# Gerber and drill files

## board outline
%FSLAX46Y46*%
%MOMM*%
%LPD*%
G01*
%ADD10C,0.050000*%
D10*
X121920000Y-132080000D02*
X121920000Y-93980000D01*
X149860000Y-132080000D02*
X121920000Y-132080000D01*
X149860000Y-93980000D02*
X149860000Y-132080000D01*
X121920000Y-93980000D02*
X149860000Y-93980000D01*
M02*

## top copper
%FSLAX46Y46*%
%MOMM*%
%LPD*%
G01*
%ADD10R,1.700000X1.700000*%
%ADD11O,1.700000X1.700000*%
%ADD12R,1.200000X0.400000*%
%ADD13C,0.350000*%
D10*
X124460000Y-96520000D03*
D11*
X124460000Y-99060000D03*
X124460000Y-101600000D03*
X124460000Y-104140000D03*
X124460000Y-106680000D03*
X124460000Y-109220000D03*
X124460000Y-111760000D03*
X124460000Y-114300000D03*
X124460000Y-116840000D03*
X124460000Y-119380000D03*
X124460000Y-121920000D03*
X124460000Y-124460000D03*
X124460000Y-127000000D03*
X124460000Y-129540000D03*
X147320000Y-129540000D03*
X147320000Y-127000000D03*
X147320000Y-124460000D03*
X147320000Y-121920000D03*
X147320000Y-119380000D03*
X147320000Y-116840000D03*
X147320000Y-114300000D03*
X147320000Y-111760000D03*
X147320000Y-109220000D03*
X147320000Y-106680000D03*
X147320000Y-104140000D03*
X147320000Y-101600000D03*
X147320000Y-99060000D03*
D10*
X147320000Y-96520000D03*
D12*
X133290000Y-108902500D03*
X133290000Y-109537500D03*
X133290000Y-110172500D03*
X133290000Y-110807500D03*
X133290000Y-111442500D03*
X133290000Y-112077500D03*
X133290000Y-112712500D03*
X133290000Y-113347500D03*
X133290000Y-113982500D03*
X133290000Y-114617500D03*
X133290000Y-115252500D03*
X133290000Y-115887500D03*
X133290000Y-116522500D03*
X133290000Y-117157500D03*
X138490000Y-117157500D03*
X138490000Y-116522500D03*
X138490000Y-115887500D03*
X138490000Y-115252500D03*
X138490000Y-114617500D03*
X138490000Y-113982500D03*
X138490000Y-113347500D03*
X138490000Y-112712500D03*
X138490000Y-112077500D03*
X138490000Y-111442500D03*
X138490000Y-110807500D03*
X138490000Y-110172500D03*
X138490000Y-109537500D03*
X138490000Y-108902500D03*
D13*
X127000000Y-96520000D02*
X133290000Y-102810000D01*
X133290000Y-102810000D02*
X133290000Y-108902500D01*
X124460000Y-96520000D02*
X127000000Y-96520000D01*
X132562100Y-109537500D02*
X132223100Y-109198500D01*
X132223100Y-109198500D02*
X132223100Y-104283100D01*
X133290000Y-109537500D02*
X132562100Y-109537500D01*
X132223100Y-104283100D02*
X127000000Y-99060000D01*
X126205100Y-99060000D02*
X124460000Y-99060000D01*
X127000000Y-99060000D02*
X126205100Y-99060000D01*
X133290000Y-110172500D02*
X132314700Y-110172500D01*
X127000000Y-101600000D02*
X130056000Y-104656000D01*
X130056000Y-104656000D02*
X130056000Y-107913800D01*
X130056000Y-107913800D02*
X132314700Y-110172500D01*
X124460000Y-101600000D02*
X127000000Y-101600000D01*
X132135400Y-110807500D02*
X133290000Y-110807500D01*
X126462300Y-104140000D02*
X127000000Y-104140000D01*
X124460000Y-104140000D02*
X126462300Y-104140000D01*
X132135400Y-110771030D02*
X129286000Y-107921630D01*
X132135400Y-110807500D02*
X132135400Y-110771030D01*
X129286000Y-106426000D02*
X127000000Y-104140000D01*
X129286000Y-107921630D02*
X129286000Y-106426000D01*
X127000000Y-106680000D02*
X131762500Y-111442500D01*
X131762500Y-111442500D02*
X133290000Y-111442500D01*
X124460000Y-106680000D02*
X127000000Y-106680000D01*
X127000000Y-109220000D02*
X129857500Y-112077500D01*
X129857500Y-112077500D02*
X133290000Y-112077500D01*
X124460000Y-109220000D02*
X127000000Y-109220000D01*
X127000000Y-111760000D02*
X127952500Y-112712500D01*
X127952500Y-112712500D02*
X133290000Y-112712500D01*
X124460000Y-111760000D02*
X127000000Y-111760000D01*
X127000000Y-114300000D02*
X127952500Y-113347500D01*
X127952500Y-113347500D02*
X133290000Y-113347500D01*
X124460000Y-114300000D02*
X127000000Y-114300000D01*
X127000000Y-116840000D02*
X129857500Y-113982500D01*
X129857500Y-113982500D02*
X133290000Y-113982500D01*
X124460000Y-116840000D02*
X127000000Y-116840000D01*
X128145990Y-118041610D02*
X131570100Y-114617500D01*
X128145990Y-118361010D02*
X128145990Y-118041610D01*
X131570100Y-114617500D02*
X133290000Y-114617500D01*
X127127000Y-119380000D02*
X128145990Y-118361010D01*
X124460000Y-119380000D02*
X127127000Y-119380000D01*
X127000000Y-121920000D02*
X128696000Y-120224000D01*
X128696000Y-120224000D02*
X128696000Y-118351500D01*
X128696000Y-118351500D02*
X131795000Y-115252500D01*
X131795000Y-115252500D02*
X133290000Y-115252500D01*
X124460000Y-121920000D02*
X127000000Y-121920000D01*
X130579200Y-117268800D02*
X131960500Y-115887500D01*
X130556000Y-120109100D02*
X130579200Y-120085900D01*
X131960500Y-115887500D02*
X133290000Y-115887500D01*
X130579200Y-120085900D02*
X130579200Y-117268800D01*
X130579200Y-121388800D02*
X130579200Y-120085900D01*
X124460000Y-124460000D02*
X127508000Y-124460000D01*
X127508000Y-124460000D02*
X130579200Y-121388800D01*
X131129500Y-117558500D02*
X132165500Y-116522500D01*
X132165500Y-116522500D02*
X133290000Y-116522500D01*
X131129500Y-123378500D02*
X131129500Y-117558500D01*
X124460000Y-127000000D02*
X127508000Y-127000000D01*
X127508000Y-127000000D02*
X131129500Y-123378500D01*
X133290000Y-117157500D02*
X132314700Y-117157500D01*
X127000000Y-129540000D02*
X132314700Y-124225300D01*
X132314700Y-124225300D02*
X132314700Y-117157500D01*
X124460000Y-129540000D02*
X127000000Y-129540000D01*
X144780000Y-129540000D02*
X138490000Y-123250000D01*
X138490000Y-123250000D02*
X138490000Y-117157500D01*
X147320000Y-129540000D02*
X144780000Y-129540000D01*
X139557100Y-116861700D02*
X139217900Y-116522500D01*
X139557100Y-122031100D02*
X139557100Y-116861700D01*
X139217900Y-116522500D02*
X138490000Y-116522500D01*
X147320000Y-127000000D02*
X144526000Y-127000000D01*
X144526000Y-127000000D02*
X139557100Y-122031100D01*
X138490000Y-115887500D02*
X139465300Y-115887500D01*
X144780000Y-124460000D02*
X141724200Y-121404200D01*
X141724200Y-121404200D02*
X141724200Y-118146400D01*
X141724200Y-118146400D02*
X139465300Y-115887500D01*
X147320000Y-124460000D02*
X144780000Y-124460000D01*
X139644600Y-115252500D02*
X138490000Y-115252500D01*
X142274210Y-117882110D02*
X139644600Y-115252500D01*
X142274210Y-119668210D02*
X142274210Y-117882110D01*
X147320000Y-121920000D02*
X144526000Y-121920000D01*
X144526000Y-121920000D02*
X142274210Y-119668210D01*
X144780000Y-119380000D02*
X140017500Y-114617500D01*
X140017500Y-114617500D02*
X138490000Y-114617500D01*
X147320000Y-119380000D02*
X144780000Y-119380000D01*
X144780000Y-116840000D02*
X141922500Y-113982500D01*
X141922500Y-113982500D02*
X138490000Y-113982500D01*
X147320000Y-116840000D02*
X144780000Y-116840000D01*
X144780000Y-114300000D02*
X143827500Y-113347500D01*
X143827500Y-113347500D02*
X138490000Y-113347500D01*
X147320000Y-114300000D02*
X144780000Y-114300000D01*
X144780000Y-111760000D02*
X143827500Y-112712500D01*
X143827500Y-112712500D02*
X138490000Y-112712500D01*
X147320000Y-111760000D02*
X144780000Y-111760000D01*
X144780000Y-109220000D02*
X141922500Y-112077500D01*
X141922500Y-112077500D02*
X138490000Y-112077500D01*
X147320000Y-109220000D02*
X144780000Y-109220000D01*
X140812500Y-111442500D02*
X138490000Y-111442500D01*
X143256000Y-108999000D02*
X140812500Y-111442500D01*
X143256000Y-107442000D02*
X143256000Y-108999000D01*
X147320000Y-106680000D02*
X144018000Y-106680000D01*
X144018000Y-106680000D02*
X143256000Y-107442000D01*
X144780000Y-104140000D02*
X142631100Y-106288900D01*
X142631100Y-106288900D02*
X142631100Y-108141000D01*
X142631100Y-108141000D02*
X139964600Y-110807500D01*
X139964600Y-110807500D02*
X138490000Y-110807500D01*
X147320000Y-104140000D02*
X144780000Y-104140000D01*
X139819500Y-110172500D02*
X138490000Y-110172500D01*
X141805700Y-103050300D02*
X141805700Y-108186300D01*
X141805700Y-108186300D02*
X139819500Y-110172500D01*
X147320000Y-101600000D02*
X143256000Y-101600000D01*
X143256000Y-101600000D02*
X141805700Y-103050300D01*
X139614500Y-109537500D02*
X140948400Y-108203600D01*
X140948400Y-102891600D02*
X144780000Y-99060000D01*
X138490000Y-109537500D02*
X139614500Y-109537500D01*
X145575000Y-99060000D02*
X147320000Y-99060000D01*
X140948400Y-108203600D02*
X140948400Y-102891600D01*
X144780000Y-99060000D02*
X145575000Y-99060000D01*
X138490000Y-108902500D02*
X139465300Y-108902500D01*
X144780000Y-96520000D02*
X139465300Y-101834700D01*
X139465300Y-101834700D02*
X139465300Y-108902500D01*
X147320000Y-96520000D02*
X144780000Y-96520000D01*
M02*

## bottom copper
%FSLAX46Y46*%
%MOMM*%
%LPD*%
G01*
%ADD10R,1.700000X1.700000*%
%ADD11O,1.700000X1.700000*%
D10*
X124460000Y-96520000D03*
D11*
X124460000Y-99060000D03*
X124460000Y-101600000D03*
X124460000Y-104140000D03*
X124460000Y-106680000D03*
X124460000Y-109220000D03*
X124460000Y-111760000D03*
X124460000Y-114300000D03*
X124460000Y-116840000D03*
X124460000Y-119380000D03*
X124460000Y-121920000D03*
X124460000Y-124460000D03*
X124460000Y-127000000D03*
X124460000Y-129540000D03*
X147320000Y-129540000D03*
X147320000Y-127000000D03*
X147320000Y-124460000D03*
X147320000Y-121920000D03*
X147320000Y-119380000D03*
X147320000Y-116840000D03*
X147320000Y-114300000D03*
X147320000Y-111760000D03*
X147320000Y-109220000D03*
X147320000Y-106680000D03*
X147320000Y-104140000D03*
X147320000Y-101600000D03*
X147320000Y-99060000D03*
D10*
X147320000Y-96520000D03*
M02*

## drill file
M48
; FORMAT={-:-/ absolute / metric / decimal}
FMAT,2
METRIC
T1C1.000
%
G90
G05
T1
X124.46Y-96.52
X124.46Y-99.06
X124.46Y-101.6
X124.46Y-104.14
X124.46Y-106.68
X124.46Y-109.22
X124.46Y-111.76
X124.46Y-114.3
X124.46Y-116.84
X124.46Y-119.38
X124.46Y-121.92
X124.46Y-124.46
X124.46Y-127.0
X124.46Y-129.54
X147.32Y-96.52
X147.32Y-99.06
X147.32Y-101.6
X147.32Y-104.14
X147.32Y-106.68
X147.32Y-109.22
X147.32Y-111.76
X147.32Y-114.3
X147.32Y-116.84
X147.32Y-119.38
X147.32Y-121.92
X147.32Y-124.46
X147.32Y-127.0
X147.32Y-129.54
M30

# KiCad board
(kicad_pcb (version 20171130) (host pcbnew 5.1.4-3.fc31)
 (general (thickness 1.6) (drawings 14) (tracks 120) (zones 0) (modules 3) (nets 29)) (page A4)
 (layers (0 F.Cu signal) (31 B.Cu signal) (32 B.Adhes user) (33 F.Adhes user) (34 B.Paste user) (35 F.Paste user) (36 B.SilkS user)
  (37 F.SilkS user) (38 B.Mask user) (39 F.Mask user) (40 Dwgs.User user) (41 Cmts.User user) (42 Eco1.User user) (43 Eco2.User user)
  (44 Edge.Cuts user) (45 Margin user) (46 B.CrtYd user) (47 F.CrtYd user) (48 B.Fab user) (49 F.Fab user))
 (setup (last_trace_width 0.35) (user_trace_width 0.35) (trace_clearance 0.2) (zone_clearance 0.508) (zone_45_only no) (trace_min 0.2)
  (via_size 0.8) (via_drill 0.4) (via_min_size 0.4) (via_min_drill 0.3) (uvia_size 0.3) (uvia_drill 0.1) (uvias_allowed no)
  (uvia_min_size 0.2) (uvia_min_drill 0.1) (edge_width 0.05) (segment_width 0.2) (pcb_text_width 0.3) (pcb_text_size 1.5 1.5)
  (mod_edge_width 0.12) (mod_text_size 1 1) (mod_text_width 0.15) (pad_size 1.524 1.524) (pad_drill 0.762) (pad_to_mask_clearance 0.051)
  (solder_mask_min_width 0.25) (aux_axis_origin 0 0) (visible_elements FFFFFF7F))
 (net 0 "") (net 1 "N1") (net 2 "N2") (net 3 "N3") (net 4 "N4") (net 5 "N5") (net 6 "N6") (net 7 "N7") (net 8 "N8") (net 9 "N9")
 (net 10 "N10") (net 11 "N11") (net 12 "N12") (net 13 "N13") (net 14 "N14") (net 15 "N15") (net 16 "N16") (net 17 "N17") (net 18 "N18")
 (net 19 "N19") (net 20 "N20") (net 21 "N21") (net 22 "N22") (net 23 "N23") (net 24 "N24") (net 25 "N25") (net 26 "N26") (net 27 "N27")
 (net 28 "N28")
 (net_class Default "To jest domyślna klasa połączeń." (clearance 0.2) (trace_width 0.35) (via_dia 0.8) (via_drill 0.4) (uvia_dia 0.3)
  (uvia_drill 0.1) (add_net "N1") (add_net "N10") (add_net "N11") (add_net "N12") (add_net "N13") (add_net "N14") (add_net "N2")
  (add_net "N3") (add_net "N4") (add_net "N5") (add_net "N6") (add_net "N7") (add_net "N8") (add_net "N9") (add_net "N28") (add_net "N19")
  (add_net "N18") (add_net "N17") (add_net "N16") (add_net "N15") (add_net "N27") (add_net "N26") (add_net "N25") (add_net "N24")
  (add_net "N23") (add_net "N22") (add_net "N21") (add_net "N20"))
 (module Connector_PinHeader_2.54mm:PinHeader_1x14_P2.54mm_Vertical (layer B.Cu) (at 124.46 96.52 180)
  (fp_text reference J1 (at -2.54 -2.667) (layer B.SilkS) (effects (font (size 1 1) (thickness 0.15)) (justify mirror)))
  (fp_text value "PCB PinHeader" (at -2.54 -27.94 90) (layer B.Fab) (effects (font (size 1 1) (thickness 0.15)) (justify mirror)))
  (pad 1 thru_hole rect (at 0 0 180) (size 1.7 1.7) (drill 1) (layers *.Cu *.Mask) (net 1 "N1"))
  (pad 2 thru_hole oval (at 0 -2.54 180) (size 1.7 1.7) (drill 1) (layers *.Cu *.Mask) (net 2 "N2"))
  (pad 3 thru_hole oval (at 0 -5.08 180) (size 1.7 1.7) (drill 1) (layers *.Cu *.Mask) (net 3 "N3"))
  (pad 4 thru_hole oval (at 0 -7.62 180) (size 1.7 1.7) (drill 1) (layers *.Cu *.Mask) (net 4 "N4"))
  (pad 5 thru_hole oval (at 0 -10.16 180) (size 1.7 1.7) (drill 1) (layers *.Cu *.Mask) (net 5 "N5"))
  (pad 6 thru_hole oval (at 0 -12.7 180) (size 1.7 1.7) (drill 1) (layers *.Cu *.Mask) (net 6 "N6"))
  (pad 7 thru_hole oval (at 0 -15.24 180) (size 1.7 1.7) (drill 1) (layers *.Cu *.Mask) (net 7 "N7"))
  (pad 8 thru_hole oval (at 0 -17.78 180) (size 1.7 1.7) (drill 1) (layers *.Cu *.Mask) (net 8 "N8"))
  (pad 9 thru_hole oval (at 0 -20.32 180) (size 1.7 1.7) (drill 1) (layers *.Cu *.Mask) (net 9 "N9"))
  (pad 10 thru_hole oval (at 0 -22.86 180) (size 1.7 1.7) (drill 1) (layers *.Cu *.Mask) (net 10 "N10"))
  (pad 11 thru_hole oval (at 0 -25.4 180) (size 1.7 1.7) (drill 1) (layers *.Cu *.Mask) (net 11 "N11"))
  (pad 12 thru_hole oval (at 0 -27.94 180) (size 1.7 1.7) (drill 1) (layers *.Cu *.Mask) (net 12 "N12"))
  (pad 13 thru_hole oval (at 0 -30.48 180) (size 1.7 1.7) (drill 1) (layers *.Cu *.Mask) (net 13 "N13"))
  (pad 14 thru_hole oval (at 0 -33.02 180) (size 1.7 1.7) (drill 1) (layers *.Cu *.Mask) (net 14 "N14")))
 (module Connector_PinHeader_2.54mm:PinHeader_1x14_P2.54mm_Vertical (layer B.Cu) (at 147.32 96.52 180)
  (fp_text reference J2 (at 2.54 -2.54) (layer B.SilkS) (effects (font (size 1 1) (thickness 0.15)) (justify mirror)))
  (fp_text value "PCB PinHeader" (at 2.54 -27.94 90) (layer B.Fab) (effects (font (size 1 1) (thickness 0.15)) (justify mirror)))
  (pad 14 thru_hole oval (at 0 -33.02 180) (size 1.7 1.7) (drill 1) (layers *.Cu *.Mask) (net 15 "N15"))
  (pad 13 thru_hole oval (at 0 -30.48 180) (size 1.7 1.7) (drill 1) (layers *.Cu *.Mask) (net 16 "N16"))
  (pad 12 thru_hole oval (at 0 -27.94 180) (size 1.7 1.7) (drill 1) (layers *.Cu *.Mask) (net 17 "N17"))
  (pad 11 thru_hole oval (at 0 -25.4 180) (size 1.7 1.7) (drill 1) (layers *.Cu *.Mask) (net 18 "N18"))
  (pad 10 thru_hole oval (at 0 -22.86 180) (size 1.7 1.7) (drill 1) (layers *.Cu *.Mask) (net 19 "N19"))
  (pad 9 thru_hole oval (at 0 -20.32 180) (size 1.7 1.7) (drill 1) (layers *.Cu *.Mask) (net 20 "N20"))
  (pad 8 thru_hole oval (at 0 -17.78 180) (size 1.7 1.7) (drill 1) (layers *.Cu *.Mask) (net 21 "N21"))
  (pad 7 thru_hole oval (at 0 -15.24 180) (size 1.7 1.7) (drill 1) (layers *.Cu *.Mask) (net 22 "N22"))
  (pad 6 thru_hole oval (at 0 -12.7 180) (size 1.7 1.7) (drill 1) (layers *.Cu *.Mask) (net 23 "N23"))
  (pad 5 thru_hole oval (at 0 -10.16 180) (size 1.7 1.7) (drill 1) (layers *.Cu *.Mask) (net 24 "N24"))
  (pad 4 thru_hole oval (at 0 -7.62 180) (size 1.7 1.7) (drill 1) (layers *.Cu *.Mask) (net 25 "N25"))
  (pad 3 thru_hole oval (at 0 -5.08 180) (size 1.7 1.7) (drill 1) (layers *.Cu *.Mask) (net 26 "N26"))
  (pad 2 thru_hole oval (at 0 -2.54 180) (size 1.7 1.7) (drill 1) (layers *.Cu *.Mask) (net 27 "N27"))
  (pad 1 thru_hole rect (at 0 0 180) (size 1.7 1.7) (drill 1) (layers *.Cu *.Mask) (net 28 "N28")))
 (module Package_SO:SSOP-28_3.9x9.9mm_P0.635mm (layer F.Cu) (at 135.89 113.03)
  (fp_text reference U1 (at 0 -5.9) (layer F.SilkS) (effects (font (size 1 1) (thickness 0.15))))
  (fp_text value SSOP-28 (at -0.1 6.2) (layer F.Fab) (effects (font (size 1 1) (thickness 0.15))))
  (pad 1 smd rect (at -2.6 -4.1275) (size 1.2 0.4) (layers F.Cu F.Paste F.Mask) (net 1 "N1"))
  (pad 2 smd rect (at -2.6 -3.4925) (size 1.2 0.4) (layers F.Cu F.Paste F.Mask) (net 2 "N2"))
  (pad 3 smd rect (at -2.6 -2.8575) (size 1.2 0.4) (layers F.Cu F.Paste F.Mask) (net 3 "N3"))
  (pad 4 smd rect (at -2.6 -2.2225) (size 1.2 0.4) (layers F.Cu F.Paste F.Mask) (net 4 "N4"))
  (pad 5 smd rect (at -2.6 -1.5875) (size 1.2 0.4) (layers F.Cu F.Paste F.Mask) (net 5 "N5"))
  (pad 6 smd rect (at -2.6 -0.9525) (size 1.2 0.4) (layers F.Cu F.Paste F.Mask) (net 6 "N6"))
  (pad 7 smd rect (at -2.6 -0.3175) (size 1.2 0.4) (layers F.Cu F.Paste F.Mask) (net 7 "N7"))
  (pad 8 smd rect (at -2.6 0.3175) (size 1.2 0.4) (layers F.Cu F.Paste F.Mask) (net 8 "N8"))
  (pad 9 smd rect (at -2.6 0.9525) (size 1.2 0.4) (layers F.Cu F.Paste F.Mask) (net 9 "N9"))
  (pad 10 smd rect (at -2.6 1.5875) (size 1.2 0.4) (layers F.Cu F.Paste F.Mask) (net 10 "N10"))
  (pad 11 smd rect (at -2.6 2.2225) (size 1.2 0.4) (layers F.Cu F.Paste F.Mask) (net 11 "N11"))
  (pad 12 smd rect (at -2.6 2.8575) (size 1.2 0.4) (layers F.Cu F.Paste F.Mask) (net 12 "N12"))
  (pad 13 smd rect (at -2.6 3.4925) (size 1.2 0.4) (layers F.Cu F.Paste F.Mask) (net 13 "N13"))
  (pad 14 smd rect (at -2.6 4.1275) (size 1.2 0.4) (layers F.Cu F.Paste F.Mask) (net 14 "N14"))
  (pad 15 smd rect (at 2.6 4.1275) (size 1.2 0.4) (layers F.Cu F.Paste F.Mask) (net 15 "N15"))
  (pad 16 smd rect (at 2.6 3.4925) (size 1.2 0.4) (layers F.Cu F.Paste F.Mask) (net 16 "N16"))
  (pad 17 smd rect (at 2.6 2.8575) (size 1.2 0.4) (layers F.Cu F.Paste F.Mask) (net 17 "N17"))
  (pad 18 smd rect (at 2.6 2.2225) (size 1.2 0.4) (layers F.Cu F.Paste F.Mask) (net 18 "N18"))
  (pad 19 smd rect (at 2.6 1.5875) (size 1.2 0.4) (layers F.Cu F.Paste F.Mask) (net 19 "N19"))
  (pad 20 smd rect (at 2.6 0.9525) (size 1.2 0.4) (layers F.Cu F.Paste F.Mask) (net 20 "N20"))
  (pad 21 smd rect (at 2.6 0.3175) (size 1.2 0.4) (layers F.Cu F.Paste F.Mask) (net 21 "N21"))
  (pad 22 smd rect (at 2.6 -0.3175) (size 1.2 0.4) (layers F.Cu F.Paste F.Mask) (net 22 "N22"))
  (pad 23 smd rect (at 2.6 -0.9525) (size 1.2 0.4) (layers F.Cu F.Paste F.Mask) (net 23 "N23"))
  (pad 24 smd rect (at 2.6 -1.5875) (size 1.2 0.4) (layers F.Cu F.Paste F.Mask) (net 24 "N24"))
  (pad 25 smd rect (at 2.6 -2.2225) (size 1.2 0.4) (layers F.Cu F.Paste F.Mask) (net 25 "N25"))
  (pad 26 smd rect (at 2.6 -2.8575) (size 1.2 0.4) (layers F.Cu F.Paste F.Mask) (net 26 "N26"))
  (pad 27 smd rect (at 2.6 -3.4925) (size 1.2 0.4) (layers F.Cu F.Paste F.Mask) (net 27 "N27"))
  (pad 28 smd rect (at 2.6 -4.1275) (size 1.2 0.4) (layers F.Cu F.Paste F.Mask) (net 28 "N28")))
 (gr_line (start 121.92 132.08) (end 121.92 93.98) (layer Edge.Cuts) (width 0.05))
 (gr_line (start 149.86 132.08) (end 121.92 132.08) (layer Edge.Cuts) (width 0.05))
 (gr_line (start 149.86 93.98) (end 149.86 132.08) (layer Edge.Cuts) (width 0.05))
 (gr_line (start 121.92 93.98) (end 149.86 93.98) (layer Edge.Cuts) (width 0.05))
 (segment (start 127 96.52) (end 133.29 102.81) (width 0.35) (layer F.Cu) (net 1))
 (segment (start 133.29 102.81) (end 133.29 108.9025) (width 0.35) (layer F.Cu) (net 1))
 (segment (start 124.46 96.52) (end 127 96.52) (width 0.35) (layer F.Cu) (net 1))
 (segment (start 132.5621 109.5375) (end 132.2231 109.1985) (width 0.35) (layer F.Cu) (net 2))
 (segment (start 132.2231 109.1985) (end 132.2231 104.2831) (width 0.35) (layer F.Cu) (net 2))
 (segment (start 133.29 109.5375) (end 132.5621 109.5375) (width 0.35) (layer F.Cu) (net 2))
 (segment (start 132.2231 104.2831) (end 127 99.06) (width 0.35) (layer F.Cu) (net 2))
 (segment (start 126.2051 99.06) (end 124.46 99.06) (width 0.35) (layer F.Cu) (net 2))
 (segment (start 127 99.06) (end 126.2051 99.06) (width 0.35) (layer F.Cu) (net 2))
 (segment (start 133.29 110.1725) (end 132.3147 110.1725) (width 0.35) (layer F.Cu) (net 3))
 (segment (start 127 101.6) (end 130.056 104.656) (width 0.35) (layer F.Cu) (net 3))
 (segment (start 130.056 104.656) (end 130.056 107.9138) (width 0.35) (layer F.Cu) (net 3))
 (segment (start 130.056 107.9138) (end 132.3147 110.1725) (width 0.35) (layer F.Cu) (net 3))
 (segment (start 124.46 101.6) (end 127 101.6) (width 0.35) (layer F.Cu) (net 3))
 (segment (start 132.1354 110.8075) (end 133.29 110.8075) (width 0.35) (layer F.Cu) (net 4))
 (segment (start 126.4623 104.14) (end 127 104.14) (width 0.35) (layer F.Cu) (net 4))
 (segment (start 124.46 104.14) (end 126.4623 104.14) (width 0.35) (layer F.Cu) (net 4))
 (segment (start 132.1354 110.77103) (end 129.286 107.92163) (width 0.35) (layer F.Cu) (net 4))
 (segment (start 132.1354 110.8075) (end 132.1354 110.77103) (width 0.35) (layer F.Cu) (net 4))
 (segment (start 129.286 106.426) (end 127 104.14) (width 0.35) (layer F.Cu) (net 4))
 (segment (start 129.286 107.92163) (end 129.286 106.426) (width 0.35) (layer F.Cu) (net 4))
 (segment (start 127 106.68) (end 131.7625 111.4425) (width 0.35) (layer F.Cu) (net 5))
 (segment (start 131.7625 111.4425) (end 133.29 111.4425) (width 0.35) (layer F.Cu) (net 5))
 (segment (start 124.46 106.68) (end 127 106.68) (width 0.35) (layer F.Cu) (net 5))
 (segment (start 127 109.22) (end 129.8575 112.0775) (width 0.35) (layer F.Cu) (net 6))
 (segment (start 129.8575 112.0775) (end 133.29 112.0775) (width 0.35) (layer F.Cu) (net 6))
 (segment (start 124.46 109.22) (end 127 109.22) (width 0.35) (layer F.Cu) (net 6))
 (segment (start 127 111.76) (end 127.9525 112.7125) (width 0.35) (layer F.Cu) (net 7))
 (segment (start 127.9525 112.7125) (end 133.29 112.7125) (width 0.35) (layer F.Cu) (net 7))
 (segment (start 124.46 111.76) (end 127 111.76) (width 0.35) (layer F.Cu) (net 7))
 (segment (start 127 114.3) (end 127.9525 113.3475) (width 0.35) (layer F.Cu) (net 8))
 (segment (start 127.9525 113.3475) (end 133.29 113.3475) (width 0.35) (layer F.Cu) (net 8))
 (segment (start 124.46 114.3) (end 127 114.3) (width 0.35) (layer F.Cu) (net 8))
 (segment (start 127 116.84) (end 129.8575 113.9825) (width 0.35) (layer F.Cu) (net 9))
 (segment (start 129.8575 113.9825) (end 133.29 113.9825) (width 0.35) (layer F.Cu) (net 9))
 (segment (start 124.46 116.84) (end 127 116.84) (width 0.35) (layer F.Cu) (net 9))
 (segment (start 128.14599 118.04161) (end 131.5701 114.6175) (width 0.35) (layer F.Cu) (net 10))
 (segment (start 128.14599 118.36101) (end 128.14599 118.04161) (width 0.35) (layer F.Cu) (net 10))
 (segment (start 131.5701 114.6175) (end 133.29 114.6175) (width 0.35) (layer F.Cu) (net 10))
 (segment (start 127.127 119.38) (end 128.14599 118.36101) (width 0.35) (layer F.Cu) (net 10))
 (segment (start 124.46 119.38) (end 127.127 119.38) (width 0.35) (layer F.Cu) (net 10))
 (segment (start 127 121.92) (end 128.696 120.224) (width 0.35) (layer F.Cu) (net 11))
 (segment (start 128.696 120.224) (end 128.696 118.3515) (width 0.35) (layer F.Cu) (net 11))
 (segment (start 128.696 118.3515) (end 131.795 115.2525) (width 0.35) (layer F.Cu) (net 11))
 (segment (start 131.795 115.2525) (end 133.29 115.2525) (width 0.35) (layer F.Cu) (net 11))
 (segment (start 124.46 121.92) (end 127 121.92) (width 0.35) (layer F.Cu) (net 11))
 (segment (start 130.5792 117.2688) (end 131.9605 115.8875) (width 0.35) (layer F.Cu) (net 12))
 (segment (start 130.556 120.1091) (end 130.5792 120.0859) (width 0.35) (layer F.Cu) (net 12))
 (segment (start 131.9605 115.8875) (end 133.29 115.8875) (width 0.35) (layer F.Cu) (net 12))
 (segment (start 130.5792 120.0859) (end 130.5792 117.2688) (width 0.35) (layer F.Cu) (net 12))
 (segment (start 130.5792 121.3888) (end 130.5792 120.0859) (width 0.35) (layer F.Cu) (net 12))
 (segment (start 124.46 124.46) (end 127.508 124.46) (width 0.35) (layer F.Cu) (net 12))
 (segment (start 127.508 124.46) (end 130.5792 121.3888) (width 0.35) (layer F.Cu) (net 12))
 (segment (start 131.1295 117.5585) (end 132.1655 116.5225) (width 0.35) (layer F.Cu) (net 13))
 (segment (start 132.1655 116.5225) (end 133.29 116.5225) (width 0.35) (layer F.Cu) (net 13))
 (segment (start 131.1295 123.3785) (end 131.1295 117.5585) (width 0.35) (layer F.Cu) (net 13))
 (segment (start 124.46 127) (end 127.508 127) (width 0.35) (layer F.Cu) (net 13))
 (segment (start 127.508 127) (end 131.1295 123.3785) (width 0.35) (layer F.Cu) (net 13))
 (segment (start 133.29 117.1575) (end 132.3147 117.1575) (width 0.35) (layer F.Cu) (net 14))
 (segment (start 127 129.54) (end 132.3147 124.2253) (width 0.35) (layer F.Cu) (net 14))
 (segment (start 132.3147 124.2253) (end 132.3147 117.1575) (width 0.35) (layer F.Cu) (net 14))
 (segment (start 124.46 129.54) (end 127 129.54) (width 0.35) (layer F.Cu) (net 14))
 (segment (start 144.78 129.54) (end 138.49 123.25) (width 0.35) (layer F.Cu) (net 15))
 (segment (start 138.49 123.25) (end 138.49 117.1575) (width 0.35) (layer F.Cu) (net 15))
 (segment (start 147.32 129.54) (end 144.78 129.54) (width 0.35) (layer F.Cu) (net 15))
 (segment (start 139.5571 116.8617) (end 139.2179 116.5225) (width 0.35) (layer F.Cu) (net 16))
 (segment (start 139.5571 122.0311) (end 139.5571 116.8617) (width 0.35) (layer F.Cu) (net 16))
 (segment (start 139.2179 116.5225) (end 138.49 116.5225) (width 0.35) (layer F.Cu) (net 16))
 (segment (start 147.32 127) (end 144.526 127) (width 0.35) (layer F.Cu) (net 16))
 (segment (start 144.526 127) (end 139.5571 122.0311) (width 0.35) (layer F.Cu) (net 16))
 (segment (start 138.49 115.8875) (end 139.4653 115.8875) (width 0.35) (layer F.Cu) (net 17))
 (segment (start 144.78 124.46) (end 141.7242 121.4042) (width 0.35) (layer F.Cu) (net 17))
 (segment (start 141.7242 121.4042) (end 141.7242 118.1464) (width 0.35) (layer F.Cu) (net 17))
 (segment (start 141.7242 118.1464) (end 139.4653 115.8875) (width 0.35) (layer F.Cu) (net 17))
 (segment (start 147.32 124.46) (end 144.78 124.46) (width 0.35) (layer F.Cu) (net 17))
 (segment (start 139.6446 115.2525) (end 138.49 115.2525) (width 0.35) (layer F.Cu) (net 18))
 (segment (start 142.27421 117.88211) (end 139.6446 115.2525) (width 0.35) (layer F.Cu) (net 18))
 (segment (start 142.27421 119.66821) (end 142.27421 117.88211) (width 0.35) (layer F.Cu) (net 18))
 (segment (start 147.32 121.92) (end 144.526 121.92) (width 0.35) (layer F.Cu) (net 18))
 (segment (start 144.526 121.92) (end 142.27421 119.66821) (width 0.35) (layer F.Cu) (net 18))
 (segment (start 144.78 119.38) (end 140.0175 114.6175) (width 0.35) (layer F.Cu) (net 19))
 (segment (start 140.0175 114.6175) (end 138.49 114.6175) (width 0.35) (layer F.Cu) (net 19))
 (segment (start 147.32 119.38) (end 144.78 119.38) (width 0.35) (layer F.Cu) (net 19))
 (segment (start 144.78 116.84) (end 141.9225 113.9825) (width 0.35) (layer F.Cu) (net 20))
 (segment (start 141.9225 113.9825) (end 138.49 113.9825) (width 0.35) (layer F.Cu) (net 20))
 (segment (start 147.32 116.84) (end 144.78 116.84) (width 0.35) (layer F.Cu) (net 20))
 (segment (start 144.78 114.3) (end 143.8275 113.3475) (width 0.35) (layer F.Cu) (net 21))
 (segment (start 143.8275 113.3475) (end 138.49 113.3475) (width 0.35) (layer F.Cu) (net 21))
 (segment (start 147.32 114.3) (end 144.78 114.3) (width 0.35) (layer F.Cu) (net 21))
 (segment (start 144.78 111.76) (end 143.8275 112.7125) (width 0.35) (layer F.Cu) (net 22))
 (segment (start 143.8275 112.7125) (end 138.49 112.7125) (width 0.35) (layer F.Cu) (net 22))
 (segment (start 147.32 111.76) (end 144.78 111.76) (width 0.35) (layer F.Cu) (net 22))
 (segment (start 144.78 109.22) (end 141.9225 112.0775) (width 0.35) (layer F.Cu) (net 23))
 (segment (start 141.9225 112.0775) (end 138.49 112.0775) (width 0.35) (layer F.Cu) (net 23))
 (segment (start 147.32 109.22) (end 144.78 109.22) (width 0.35) (layer F.Cu) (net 23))
 (segment (start 140.8125 111.4425) (end 138.49 111.4425) (width 0.35) (layer F.Cu) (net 24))
 (segment (start 143.256 108.999) (end 140.8125 111.4425) (width 0.35) (layer F.Cu) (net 24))
 (segment (start 143.256 107.442) (end 143.256 108.999) (width 0.35) (layer F.Cu) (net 24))
 (segment (start 147.32 106.68) (end 144.018 106.68) (width 0.35) (layer F.Cu) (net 24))
 (segment (start 144.018 106.68) (end 143.256 107.442) (width 0.35) (layer F.Cu) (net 24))
 (segment (start 144.78 104.14) (end 142.6311 106.2889) (width 0.35) (layer F.Cu) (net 25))
 (segment (start 142.6311 106.2889) (end 142.6311 108.141) (width 0.35) (layer F.Cu) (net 25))
 (segment (start 142.6311 108.141) (end 139.9646 110.8075) (width 0.35) (layer F.Cu) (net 25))
 (segment (start 139.9646 110.8075) (end 138.49 110.8075) (width 0.35) (layer F.Cu) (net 25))
 (segment (start 147.32 104.14) (end 144.78 104.14) (width 0.35) (layer F.Cu) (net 25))
 (segment (start 139.8195 110.1725) (end 138.49 110.1725) (width 0.35) (layer F.Cu) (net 26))
 (segment (start 141.8057 103.0503) (end 141.8057 108.1863) (width 0.35) (layer F.Cu) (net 26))
 (segment (start 141.8057 108.1863) (end 139.8195 110.1725) (width 0.35) (layer F.Cu) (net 26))
 (segment (start 147.32 101.6) (end 143.256 101.6) (width 0.35) (layer F.Cu) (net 26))
 (segment (start 143.256 101.6) (end 141.8057 103.0503) (width 0.35) (layer F.Cu) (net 26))
 (segment (start 139.6145 109.5375) (end 140.9484 108.2036) (width 0.35) (layer F.Cu) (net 27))
 (segment (start 140.9484 102.8916) (end 144.78 99.06) (width 0.35) (layer F.Cu) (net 27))
 (segment (start 138.49 109.5375) (end 139.6145 109.5375) (width 0.35) (layer F.Cu) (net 27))
 (segment (start 145.575 99.06) (end 147.32 99.06) (width 0.35) (layer F.Cu) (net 27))
 (segment (start 140.9484 108.2036) (end 140.9484 102.8916) (width 0.35) (layer F.Cu) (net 27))
 (segment (start 144.78 99.06) (end 145.575 99.06) (width 0.35) (layer F.Cu) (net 27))
 (segment (start 138.49 108.9025) (end 139.4653 108.9025) (width 0.35) (layer F.Cu) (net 28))
 (segment (start 144.78 96.52) (end 139.4653 101.8347) (width 0.35) (layer F.Cu) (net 28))
 (segment (start 139.4653 101.8347) (end 139.4653 108.9025) (width 0.35) (layer F.Cu) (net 28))
 (segment (start 147.32 96.52) (end 144.78 96.52) (width 0.35) (layer F.Cu) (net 28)))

